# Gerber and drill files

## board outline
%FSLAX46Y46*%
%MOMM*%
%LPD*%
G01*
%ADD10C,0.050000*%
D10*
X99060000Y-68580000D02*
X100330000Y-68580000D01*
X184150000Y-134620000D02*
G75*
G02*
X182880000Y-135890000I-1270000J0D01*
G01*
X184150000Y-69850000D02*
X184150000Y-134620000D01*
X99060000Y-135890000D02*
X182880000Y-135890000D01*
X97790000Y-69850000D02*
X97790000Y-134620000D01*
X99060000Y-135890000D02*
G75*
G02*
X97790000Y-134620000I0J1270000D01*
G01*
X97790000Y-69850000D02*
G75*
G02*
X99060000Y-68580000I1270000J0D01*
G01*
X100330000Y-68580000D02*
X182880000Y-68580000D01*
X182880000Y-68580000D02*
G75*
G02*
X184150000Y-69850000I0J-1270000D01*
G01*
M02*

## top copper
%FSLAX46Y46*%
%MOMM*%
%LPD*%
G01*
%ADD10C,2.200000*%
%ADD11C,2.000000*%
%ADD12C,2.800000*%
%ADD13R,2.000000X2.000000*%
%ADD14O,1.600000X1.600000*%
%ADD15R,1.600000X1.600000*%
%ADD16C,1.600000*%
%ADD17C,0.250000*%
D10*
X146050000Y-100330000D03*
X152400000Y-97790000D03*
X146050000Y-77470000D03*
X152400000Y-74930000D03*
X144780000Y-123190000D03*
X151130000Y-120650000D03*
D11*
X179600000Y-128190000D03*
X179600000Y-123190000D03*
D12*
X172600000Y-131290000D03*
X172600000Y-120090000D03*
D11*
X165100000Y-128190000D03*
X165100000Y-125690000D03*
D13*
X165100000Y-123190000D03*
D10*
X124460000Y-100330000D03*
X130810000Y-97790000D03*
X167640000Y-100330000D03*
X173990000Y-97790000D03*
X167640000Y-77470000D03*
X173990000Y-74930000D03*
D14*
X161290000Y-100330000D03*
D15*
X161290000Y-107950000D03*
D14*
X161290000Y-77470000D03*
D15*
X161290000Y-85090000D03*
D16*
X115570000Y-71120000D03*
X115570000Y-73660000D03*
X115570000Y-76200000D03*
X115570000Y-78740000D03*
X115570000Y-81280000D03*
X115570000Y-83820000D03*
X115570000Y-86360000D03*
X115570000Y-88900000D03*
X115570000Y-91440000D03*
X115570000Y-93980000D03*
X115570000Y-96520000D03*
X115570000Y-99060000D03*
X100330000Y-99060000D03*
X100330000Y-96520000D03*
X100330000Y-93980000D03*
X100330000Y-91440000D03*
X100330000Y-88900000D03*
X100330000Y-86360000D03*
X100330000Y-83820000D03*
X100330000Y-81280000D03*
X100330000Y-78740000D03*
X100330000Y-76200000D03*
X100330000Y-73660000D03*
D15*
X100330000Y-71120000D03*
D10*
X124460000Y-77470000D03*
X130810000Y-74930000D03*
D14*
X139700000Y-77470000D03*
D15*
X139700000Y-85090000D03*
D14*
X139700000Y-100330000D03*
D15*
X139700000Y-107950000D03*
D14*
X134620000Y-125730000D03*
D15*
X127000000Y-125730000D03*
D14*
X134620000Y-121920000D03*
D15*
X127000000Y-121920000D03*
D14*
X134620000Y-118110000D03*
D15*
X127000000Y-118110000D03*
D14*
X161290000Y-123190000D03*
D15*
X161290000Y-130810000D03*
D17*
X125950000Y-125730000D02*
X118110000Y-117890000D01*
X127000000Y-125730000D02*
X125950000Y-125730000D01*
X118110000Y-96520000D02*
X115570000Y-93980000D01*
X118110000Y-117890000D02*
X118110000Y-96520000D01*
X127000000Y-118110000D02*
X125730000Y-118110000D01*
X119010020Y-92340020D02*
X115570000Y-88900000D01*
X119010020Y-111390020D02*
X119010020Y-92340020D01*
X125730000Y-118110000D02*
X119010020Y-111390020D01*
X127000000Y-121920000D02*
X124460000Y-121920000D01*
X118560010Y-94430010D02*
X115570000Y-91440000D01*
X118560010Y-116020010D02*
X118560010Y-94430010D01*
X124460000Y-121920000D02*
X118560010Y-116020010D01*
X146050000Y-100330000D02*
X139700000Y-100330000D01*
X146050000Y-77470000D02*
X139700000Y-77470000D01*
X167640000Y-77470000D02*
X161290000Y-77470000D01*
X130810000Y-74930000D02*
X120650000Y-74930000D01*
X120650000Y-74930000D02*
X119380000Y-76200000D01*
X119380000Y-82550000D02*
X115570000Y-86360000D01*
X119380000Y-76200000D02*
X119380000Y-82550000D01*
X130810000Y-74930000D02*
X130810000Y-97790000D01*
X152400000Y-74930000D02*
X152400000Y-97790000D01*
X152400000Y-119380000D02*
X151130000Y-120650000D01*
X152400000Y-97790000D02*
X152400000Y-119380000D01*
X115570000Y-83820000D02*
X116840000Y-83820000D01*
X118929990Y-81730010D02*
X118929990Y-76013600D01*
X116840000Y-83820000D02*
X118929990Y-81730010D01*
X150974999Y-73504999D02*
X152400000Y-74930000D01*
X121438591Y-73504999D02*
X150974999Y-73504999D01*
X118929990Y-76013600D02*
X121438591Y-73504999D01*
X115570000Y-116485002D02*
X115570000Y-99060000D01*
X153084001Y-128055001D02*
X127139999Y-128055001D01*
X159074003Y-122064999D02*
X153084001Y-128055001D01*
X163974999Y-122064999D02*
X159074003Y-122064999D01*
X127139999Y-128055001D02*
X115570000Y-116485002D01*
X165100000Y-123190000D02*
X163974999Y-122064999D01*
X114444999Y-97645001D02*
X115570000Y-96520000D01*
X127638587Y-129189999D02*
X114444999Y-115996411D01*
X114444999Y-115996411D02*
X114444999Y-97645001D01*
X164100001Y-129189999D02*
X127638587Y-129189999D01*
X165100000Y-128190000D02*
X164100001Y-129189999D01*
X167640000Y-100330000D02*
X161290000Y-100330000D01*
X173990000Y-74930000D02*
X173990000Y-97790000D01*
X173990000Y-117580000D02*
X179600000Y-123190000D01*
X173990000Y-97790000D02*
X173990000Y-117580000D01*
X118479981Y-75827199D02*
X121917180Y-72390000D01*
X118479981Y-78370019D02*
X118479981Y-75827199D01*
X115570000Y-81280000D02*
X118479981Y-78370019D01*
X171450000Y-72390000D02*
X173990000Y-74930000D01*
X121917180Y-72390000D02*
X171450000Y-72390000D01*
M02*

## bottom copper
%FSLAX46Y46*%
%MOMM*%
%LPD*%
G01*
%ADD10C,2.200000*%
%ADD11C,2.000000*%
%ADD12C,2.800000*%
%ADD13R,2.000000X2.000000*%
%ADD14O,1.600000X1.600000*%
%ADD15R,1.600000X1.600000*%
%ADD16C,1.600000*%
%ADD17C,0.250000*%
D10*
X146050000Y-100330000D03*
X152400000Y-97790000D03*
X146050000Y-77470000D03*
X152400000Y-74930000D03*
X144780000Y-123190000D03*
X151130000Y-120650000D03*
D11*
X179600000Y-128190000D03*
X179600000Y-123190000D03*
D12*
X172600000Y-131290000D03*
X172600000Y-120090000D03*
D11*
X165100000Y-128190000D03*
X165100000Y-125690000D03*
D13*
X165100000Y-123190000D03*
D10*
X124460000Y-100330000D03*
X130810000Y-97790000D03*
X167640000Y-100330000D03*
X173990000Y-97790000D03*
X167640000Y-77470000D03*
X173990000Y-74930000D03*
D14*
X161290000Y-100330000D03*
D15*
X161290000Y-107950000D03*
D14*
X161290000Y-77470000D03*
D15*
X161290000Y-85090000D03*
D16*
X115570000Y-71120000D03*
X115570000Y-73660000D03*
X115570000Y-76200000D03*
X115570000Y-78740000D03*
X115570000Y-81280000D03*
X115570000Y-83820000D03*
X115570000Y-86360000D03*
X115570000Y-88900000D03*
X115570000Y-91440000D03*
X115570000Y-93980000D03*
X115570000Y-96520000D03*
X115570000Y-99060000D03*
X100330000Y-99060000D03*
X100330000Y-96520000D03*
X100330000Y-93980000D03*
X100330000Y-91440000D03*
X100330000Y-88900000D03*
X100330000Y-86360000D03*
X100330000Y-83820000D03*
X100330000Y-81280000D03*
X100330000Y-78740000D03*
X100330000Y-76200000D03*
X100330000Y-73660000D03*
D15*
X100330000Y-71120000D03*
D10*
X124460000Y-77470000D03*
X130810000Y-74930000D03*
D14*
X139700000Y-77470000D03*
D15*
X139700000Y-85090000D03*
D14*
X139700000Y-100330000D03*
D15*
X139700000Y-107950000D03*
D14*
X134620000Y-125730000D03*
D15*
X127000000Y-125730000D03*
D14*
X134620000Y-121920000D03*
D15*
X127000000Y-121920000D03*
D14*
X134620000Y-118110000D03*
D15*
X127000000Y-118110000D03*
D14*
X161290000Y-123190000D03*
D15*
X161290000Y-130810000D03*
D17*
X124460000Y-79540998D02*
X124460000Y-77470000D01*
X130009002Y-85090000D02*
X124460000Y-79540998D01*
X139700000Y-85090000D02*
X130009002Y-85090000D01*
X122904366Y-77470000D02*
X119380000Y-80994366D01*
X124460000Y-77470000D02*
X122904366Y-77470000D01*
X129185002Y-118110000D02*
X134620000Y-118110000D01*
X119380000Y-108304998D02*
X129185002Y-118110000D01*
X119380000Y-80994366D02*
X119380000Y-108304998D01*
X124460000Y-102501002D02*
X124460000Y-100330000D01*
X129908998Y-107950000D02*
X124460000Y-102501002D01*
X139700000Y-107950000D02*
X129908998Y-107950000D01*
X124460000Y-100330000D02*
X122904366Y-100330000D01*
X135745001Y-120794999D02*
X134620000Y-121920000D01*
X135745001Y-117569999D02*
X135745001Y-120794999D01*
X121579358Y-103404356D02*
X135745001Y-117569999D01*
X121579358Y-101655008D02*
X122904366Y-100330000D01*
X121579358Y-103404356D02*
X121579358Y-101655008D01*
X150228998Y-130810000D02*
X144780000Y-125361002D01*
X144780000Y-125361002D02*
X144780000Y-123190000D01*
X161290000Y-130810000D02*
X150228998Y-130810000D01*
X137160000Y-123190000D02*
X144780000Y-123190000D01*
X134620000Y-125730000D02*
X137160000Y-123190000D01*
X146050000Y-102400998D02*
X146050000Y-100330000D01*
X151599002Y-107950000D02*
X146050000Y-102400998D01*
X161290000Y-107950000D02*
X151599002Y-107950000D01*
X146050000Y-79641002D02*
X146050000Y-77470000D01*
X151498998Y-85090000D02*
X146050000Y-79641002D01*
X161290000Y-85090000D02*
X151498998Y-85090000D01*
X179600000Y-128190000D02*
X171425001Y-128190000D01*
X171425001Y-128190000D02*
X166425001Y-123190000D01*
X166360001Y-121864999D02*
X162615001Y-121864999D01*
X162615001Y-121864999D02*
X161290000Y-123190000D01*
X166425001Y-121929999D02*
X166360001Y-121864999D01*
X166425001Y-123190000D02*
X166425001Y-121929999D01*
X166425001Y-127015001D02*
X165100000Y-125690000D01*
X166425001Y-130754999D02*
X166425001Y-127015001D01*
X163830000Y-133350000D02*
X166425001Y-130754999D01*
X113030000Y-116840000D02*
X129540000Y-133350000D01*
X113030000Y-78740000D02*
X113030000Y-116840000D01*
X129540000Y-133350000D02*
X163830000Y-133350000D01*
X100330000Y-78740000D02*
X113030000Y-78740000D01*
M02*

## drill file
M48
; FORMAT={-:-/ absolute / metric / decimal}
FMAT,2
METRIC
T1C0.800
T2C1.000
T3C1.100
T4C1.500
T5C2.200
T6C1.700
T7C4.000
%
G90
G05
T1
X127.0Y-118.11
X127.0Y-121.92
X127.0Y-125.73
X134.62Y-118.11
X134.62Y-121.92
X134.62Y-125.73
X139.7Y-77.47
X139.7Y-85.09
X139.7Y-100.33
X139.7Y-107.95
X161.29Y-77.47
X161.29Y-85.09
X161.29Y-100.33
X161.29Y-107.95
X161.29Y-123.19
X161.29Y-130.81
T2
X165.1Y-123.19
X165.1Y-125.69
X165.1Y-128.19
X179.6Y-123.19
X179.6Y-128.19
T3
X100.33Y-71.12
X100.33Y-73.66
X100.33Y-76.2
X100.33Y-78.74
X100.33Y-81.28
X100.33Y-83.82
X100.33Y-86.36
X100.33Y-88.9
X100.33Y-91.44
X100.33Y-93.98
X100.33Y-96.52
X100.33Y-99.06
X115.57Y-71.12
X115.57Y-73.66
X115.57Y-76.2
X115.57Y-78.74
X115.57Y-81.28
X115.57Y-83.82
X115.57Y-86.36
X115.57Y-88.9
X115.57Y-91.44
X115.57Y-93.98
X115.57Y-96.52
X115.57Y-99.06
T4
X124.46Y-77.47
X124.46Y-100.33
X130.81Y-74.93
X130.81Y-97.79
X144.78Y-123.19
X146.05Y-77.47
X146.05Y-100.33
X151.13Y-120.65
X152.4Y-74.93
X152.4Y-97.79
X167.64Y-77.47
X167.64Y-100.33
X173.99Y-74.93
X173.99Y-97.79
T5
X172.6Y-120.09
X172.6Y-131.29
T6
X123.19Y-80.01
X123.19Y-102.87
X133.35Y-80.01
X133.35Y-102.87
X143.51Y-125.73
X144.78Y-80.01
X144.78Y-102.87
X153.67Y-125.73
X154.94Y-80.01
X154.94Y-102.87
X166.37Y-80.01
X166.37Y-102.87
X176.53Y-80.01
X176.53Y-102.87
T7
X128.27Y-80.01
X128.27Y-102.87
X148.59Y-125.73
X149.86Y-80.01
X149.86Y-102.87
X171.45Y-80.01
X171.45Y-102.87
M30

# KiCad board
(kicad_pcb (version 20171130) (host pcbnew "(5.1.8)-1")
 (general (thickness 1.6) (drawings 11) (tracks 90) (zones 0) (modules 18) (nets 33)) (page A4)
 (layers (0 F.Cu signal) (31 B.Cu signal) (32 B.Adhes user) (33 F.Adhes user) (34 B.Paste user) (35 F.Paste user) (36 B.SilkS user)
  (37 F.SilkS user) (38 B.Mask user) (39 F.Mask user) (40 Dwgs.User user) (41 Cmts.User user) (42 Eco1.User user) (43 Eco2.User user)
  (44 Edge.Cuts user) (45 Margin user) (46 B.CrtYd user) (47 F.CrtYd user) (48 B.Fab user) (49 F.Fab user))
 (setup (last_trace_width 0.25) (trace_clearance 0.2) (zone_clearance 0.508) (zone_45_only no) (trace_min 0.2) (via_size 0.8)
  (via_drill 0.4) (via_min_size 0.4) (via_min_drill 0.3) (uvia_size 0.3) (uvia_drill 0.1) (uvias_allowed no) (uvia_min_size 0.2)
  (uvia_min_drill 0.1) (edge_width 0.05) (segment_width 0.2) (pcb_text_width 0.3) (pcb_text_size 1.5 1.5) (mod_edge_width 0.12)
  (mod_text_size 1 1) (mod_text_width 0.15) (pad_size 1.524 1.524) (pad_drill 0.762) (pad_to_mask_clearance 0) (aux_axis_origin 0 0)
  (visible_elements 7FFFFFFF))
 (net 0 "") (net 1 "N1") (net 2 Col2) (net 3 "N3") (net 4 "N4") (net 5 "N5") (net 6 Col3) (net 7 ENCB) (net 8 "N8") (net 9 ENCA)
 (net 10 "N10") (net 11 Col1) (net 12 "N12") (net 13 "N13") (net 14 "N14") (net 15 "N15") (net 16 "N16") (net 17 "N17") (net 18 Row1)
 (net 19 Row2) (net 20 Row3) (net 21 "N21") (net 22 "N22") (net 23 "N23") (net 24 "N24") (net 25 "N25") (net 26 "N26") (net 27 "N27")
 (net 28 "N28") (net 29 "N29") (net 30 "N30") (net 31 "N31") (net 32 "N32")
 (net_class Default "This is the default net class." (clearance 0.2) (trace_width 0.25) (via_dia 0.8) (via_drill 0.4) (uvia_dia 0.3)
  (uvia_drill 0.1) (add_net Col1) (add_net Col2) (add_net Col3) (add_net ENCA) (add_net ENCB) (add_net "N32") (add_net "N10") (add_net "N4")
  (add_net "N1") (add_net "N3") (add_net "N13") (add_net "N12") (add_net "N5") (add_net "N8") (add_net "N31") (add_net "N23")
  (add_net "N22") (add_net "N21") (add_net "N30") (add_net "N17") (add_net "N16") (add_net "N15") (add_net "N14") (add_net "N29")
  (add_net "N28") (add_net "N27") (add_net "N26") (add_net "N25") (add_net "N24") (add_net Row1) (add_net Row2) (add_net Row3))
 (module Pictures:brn (layer F.Cu) (at 110.49 128.27)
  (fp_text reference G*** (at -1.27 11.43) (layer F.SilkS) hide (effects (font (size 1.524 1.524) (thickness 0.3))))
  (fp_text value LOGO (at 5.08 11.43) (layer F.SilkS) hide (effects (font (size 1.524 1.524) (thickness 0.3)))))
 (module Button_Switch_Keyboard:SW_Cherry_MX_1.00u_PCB (layer F.Cu) (at 152.4 97.79)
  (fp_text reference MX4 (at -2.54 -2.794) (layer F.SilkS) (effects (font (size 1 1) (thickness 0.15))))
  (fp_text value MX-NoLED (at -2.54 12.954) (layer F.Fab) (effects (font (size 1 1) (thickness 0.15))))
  (pad "" np_thru_hole circle (at 2.54 5.08) (size 1.7 1.7) (drill 1.7) (layers *.Cu *.Mask))
  (pad "" np_thru_hole circle (at -7.62 5.08) (size 1.7 1.7) (drill 1.7) (layers *.Cu *.Mask))
  (pad "" np_thru_hole circle (at -2.54 5.08) (size 4 4) (drill 4) (layers *.Cu *.Mask))
  (pad 2 thru_hole circle (at -6.35 2.54) (size 2.2 2.2) (drill 1.5) (layers *.Cu *.Mask) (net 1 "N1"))
  (pad 1 thru_hole circle (at 0 0) (size 2.2 2.2) (drill 1.5) (layers *.Cu *.Mask) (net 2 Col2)))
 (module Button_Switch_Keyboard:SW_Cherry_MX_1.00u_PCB (layer F.Cu) (at 152.4 74.93)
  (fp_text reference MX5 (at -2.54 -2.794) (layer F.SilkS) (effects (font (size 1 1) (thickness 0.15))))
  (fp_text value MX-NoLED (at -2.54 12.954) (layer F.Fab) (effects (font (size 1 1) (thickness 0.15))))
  (pad "" np_thru_hole circle (at 2.54 5.08) (size 1.7 1.7) (drill 1.7) (layers *.Cu *.Mask))
  (pad "" np_thru_hole circle (at -7.62 5.08) (size 1.7 1.7) (drill 1.7) (layers *.Cu *.Mask))
  (pad "" np_thru_hole circle (at -2.54 5.08) (size 4 4) (drill 4) (layers *.Cu *.Mask))
  (pad 2 thru_hole circle (at -6.35 2.54) (size 2.2 2.2) (drill 1.5) (layers *.Cu *.Mask) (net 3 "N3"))
  (pad 1 thru_hole circle (at 0 0) (size 2.2 2.2) (drill 1.5) (layers *.Cu *.Mask) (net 2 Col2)))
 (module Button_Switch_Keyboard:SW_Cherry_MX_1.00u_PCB (layer F.Cu) (at 151.13 120.65)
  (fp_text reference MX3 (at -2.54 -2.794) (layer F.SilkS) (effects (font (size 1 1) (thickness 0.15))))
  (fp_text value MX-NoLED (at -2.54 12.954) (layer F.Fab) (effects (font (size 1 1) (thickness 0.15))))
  (pad "" np_thru_hole circle (at 2.54 5.08) (size 1.7 1.7) (drill 1.7) (layers *.Cu *.Mask))
  (pad "" np_thru_hole circle (at -7.62 5.08) (size 1.7 1.7) (drill 1.7) (layers *.Cu *.Mask))
  (pad "" np_thru_hole circle (at -2.54 5.08) (size 4 4) (drill 4) (layers *.Cu *.Mask))
  (pad 2 thru_hole circle (at -6.35 2.54) (size 2.2 2.2) (drill 1.5) (layers *.Cu *.Mask) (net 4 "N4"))
  (pad 1 thru_hole circle (at 0 0) (size 2.2 2.2) (drill 1.5) (layers *.Cu *.Mask) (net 2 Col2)))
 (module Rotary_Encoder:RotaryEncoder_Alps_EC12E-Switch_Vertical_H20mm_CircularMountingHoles (layer F.Cu) (at 165.1 123.19)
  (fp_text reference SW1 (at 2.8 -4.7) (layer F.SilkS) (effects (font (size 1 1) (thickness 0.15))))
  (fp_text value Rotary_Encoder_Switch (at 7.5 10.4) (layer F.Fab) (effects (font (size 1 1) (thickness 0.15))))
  (pad S2 thru_hole circle (at 14.5 5) (size 2 2) (drill 1) (layers *.Cu *.Mask) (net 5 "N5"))
  (pad S1 thru_hole circle (at 14.5 0) (size 2 2) (drill 1) (layers *.Cu *.Mask) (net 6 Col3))
  (pad MP thru_hole circle (at 7.5 8.1) (size 2.8 2.8) (drill 2.2) (layers *.Cu *.Mask))
  (pad MP thru_hole circle (at 7.5 -3.1) (size 2.8 2.8) (drill 2.2) (layers *.Cu *.Mask))
  (pad B thru_hole circle (at 0 5) (size 2 2) (drill 1) (layers *.Cu *.Mask) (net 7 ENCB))
  (pad C thru_hole circle (at 0 2.5) (size 2 2) (drill 1) (layers *.Cu *.Mask) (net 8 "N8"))
  (pad A thru_hole rect (at 0 0) (size 2 2) (drill 1) (layers *.Cu *.Mask) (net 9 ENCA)))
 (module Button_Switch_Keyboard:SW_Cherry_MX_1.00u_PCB (layer F.Cu) (at 130.81 97.79)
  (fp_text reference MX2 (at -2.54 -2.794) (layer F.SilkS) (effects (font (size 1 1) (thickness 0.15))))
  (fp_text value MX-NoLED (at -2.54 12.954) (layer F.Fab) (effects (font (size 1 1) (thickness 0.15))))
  (pad "" np_thru_hole circle (at 2.54 5.08) (size 1.7 1.7) (drill 1.7) (layers *.Cu *.Mask))
  (pad "" np_thru_hole circle (at -7.62 5.08) (size 1.7 1.7) (drill 1.7) (layers *.Cu *.Mask))
  (pad "" np_thru_hole circle (at -2.54 5.08) (size 4 4) (drill 4) (layers *.Cu *.Mask))
  (pad 2 thru_hole circle (at -6.35 2.54) (size 2.2 2.2) (drill 1.5) (layers *.Cu *.Mask) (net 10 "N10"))
  (pad 1 thru_hole circle (at 0 0) (size 2.2 2.2) (drill 1.5) (layers *.Cu *.Mask) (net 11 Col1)))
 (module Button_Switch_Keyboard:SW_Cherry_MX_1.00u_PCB (layer F.Cu) (at 173.99 97.79)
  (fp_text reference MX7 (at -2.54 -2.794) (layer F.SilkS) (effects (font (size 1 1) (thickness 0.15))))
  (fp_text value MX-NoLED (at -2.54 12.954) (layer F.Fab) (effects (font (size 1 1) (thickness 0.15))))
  (pad "" np_thru_hole circle (at 2.54 5.08) (size 1.7 1.7) (drill 1.7) (layers *.Cu *.Mask))
  (pad "" np_thru_hole circle (at -7.62 5.08) (size 1.7 1.7) (drill 1.7) (layers *.Cu *.Mask))
  (pad "" np_thru_hole circle (at -2.54 5.08) (size 4 4) (drill 4) (layers *.Cu *.Mask))
  (pad 2 thru_hole circle (at -6.35 2.54) (size 2.2 2.2) (drill 1.5) (layers *.Cu *.Mask) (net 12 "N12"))
  (pad 1 thru_hole circle (at 0 0) (size 2.2 2.2) (drill 1.5) (layers *.Cu *.Mask) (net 6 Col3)))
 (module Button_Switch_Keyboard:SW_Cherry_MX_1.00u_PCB (layer F.Cu) (at 173.99 74.93)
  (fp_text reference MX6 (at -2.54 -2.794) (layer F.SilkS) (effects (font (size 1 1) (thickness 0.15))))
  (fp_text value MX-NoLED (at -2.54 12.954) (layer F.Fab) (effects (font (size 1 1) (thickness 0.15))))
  (pad "" np_thru_hole circle (at 2.54 5.08) (size 1.7 1.7) (drill 1.7) (layers *.Cu *.Mask))
  (pad "" np_thru_hole circle (at -7.62 5.08) (size 1.7 1.7) (drill 1.7) (layers *.Cu *.Mask))
  (pad "" np_thru_hole circle (at -2.54 5.08) (size 4 4) (drill 4) (layers *.Cu *.Mask))
  (pad 2 thru_hole circle (at -6.35 2.54) (size 2.2 2.2) (drill 1.5) (layers *.Cu *.Mask) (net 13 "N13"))
  (pad 1 thru_hole circle (at 0 0) (size 2.2 2.2) (drill 1.5) (layers *.Cu *.Mask) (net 6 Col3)))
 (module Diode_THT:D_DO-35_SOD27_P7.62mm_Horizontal (layer F.Cu) (at 161.29 107.95 90)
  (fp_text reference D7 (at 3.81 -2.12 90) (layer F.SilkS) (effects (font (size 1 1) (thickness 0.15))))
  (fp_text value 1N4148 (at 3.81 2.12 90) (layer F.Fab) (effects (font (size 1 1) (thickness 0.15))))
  (pad 2 thru_hole oval (at 7.62 0 90) (size 1.6 1.6) (drill 0.8) (layers *.Cu *.Mask) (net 12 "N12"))
  (pad 1 thru_hole rect (at 0 0 90) (size 1.6 1.6) (drill 0.8) (layers *.Cu *.Mask) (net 1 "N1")))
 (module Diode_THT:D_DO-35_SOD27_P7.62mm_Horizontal (layer F.Cu) (at 161.29 85.09 90)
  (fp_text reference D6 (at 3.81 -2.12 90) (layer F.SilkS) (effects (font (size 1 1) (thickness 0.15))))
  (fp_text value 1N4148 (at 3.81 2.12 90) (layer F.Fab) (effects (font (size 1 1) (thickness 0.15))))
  (pad 2 thru_hole oval (at 7.62 0 90) (size 1.6 1.6) (drill 0.8) (layers *.Cu *.Mask) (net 13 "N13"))
  (pad 1 thru_hole rect (at 0 0 90) (size 1.6 1.6) (drill 0.8) (layers *.Cu *.Mask) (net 3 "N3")))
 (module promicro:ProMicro (layer F.Cu) (at 107.95 85.09 270)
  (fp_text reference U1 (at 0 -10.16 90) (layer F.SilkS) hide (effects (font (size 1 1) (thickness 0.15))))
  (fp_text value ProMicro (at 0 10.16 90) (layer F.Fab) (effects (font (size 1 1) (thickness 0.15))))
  (pad 24 thru_hole circle (at -13.97 -7.62 270) (size 1.6 1.6) (drill 1.1) (layers *.Cu *.Mask F.SilkS) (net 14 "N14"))
  (pad 23 thru_hole circle (at -11.43 -7.62 270) (size 1.6 1.6) (drill 1.1) (layers *.Cu *.Mask F.SilkS) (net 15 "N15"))
  (pad 22 thru_hole circle (at -8.89 -7.62 270) (size 1.6 1.6) (drill 1.1) (layers *.Cu *.Mask F.SilkS) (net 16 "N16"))
  (pad 21 thru_hole circle (at -6.35 -7.62 270) (size 1.6 1.6) (drill 1.1) (layers *.Cu *.Mask F.SilkS) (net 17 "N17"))
  (pad 20 thru_hole circle (at -3.81 -7.62 270) (size 1.6 1.6) (drill 1.1) (layers *.Cu *.Mask F.SilkS) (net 6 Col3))
  (pad 19 thru_hole circle (at -1.27 -7.62 270) (size 1.6 1.6) (drill 1.1) (layers *.Cu *.Mask F.SilkS) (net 2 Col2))
  (pad 18 thru_hole circle (at 1.27 -7.62 270) (size 1.6 1.6) (drill 1.1) (layers *.Cu *.Mask F.SilkS) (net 11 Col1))
  (pad 17 thru_hole circle (at 3.81 -7.62 270) (size 1.6 1.6) (drill 1.1) (layers *.Cu *.Mask F.SilkS) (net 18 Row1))
  (pad 16 thru_hole circle (at 6.35 -7.62 270) (size 1.6 1.6) (drill 1.1) (layers *.Cu *.Mask F.SilkS) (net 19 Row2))
  (pad 15 thru_hole circle (at 8.89 -7.62 270) (size 1.6 1.6) (drill 1.1) (layers *.Cu *.Mask F.SilkS) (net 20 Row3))
  (pad 14 thru_hole circle (at 11.43 -7.62 270) (size 1.6 1.6) (drill 1.1) (layers *.Cu *.Mask F.SilkS) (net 7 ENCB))
  (pad 13 thru_hole circle (at 13.97 -7.62 270) (size 1.6 1.6) (drill 1.1) (layers *.Cu *.Mask F.SilkS) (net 9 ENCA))
  (pad 12 thru_hole circle (at 13.97 7.62 270) (size 1.6 1.6) (drill 1.1) (layers *.Cu *.Mask F.SilkS) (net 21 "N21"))
  (pad 11 thru_hole circle (at 11.43 7.62 270) (size 1.6 1.6) (drill 1.1) (layers *.Cu *.Mask F.SilkS) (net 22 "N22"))
  (pad 10 thru_hole circle (at 8.89 7.62 270) (size 1.6 1.6) (drill 1.1) (layers *.Cu *.Mask F.SilkS) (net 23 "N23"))
  (pad 9 thru_hole circle (at 6.35 7.62 270) (size 1.6 1.6) (drill 1.1) (layers *.Cu *.Mask F.SilkS) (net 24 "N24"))
  (pad 8 thru_hole circle (at 3.81 7.62 270) (size 1.6 1.6) (drill 1.1) (layers *.Cu *.Mask F.SilkS) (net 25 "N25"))
  (pad 7 thru_hole circle (at 1.27 7.62 270) (size 1.6 1.6) (drill 1.1) (layers *.Cu *.Mask F.SilkS) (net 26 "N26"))
  (pad 6 thru_hole circle (at -1.27 7.62 270) (size 1.6 1.6) (drill 1.1) (layers *.Cu *.Mask F.SilkS) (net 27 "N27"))
  (pad 5 thru_hole circle (at -3.81 7.62 270) (size 1.6 1.6) (drill 1.1) (layers *.Cu *.Mask F.SilkS) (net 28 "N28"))
  (pad 4 thru_hole circle (at -6.35 7.62 270) (size 1.6 1.6) (drill 1.1) (layers *.Cu *.Mask F.SilkS) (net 8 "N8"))
  (pad 3 thru_hole circle (at -8.89 7.62 270) (size 1.6 1.6) (drill 1.1) (layers *.Cu *.Mask F.SilkS) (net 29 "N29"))
  (pad 2 thru_hole circle (at -11.43 7.62 270) (size 1.6 1.6) (drill 1.1) (layers *.Cu *.Mask F.SilkS) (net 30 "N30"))
  (pad 1 thru_hole rect (at -13.97 7.62 270) (size 1.6 1.6) (drill 1.1) (layers *.Cu *.Mask F.SilkS) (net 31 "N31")))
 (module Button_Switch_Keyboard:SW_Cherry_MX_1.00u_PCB (layer F.Cu) (at 130.81 74.93)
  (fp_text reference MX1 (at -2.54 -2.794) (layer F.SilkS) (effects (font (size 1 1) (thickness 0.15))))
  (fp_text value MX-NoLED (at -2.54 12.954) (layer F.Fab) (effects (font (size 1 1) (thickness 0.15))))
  (pad "" np_thru_hole circle (at 2.54 5.08) (size 1.7 1.7) (drill 1.7) (layers *.Cu *.Mask))
  (pad "" np_thru_hole circle (at -7.62 5.08) (size 1.7 1.7) (drill 1.7) (layers *.Cu *.Mask))
  (pad "" np_thru_hole circle (at -2.54 5.08) (size 4 4) (drill 4) (layers *.Cu *.Mask))
  (pad 2 thru_hole circle (at -6.35 2.54) (size 2.2 2.2) (drill 1.5) (layers *.Cu *.Mask) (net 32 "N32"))
  (pad 1 thru_hole circle (at 0 0) (size 2.2 2.2) (drill 1.5) (layers *.Cu *.Mask) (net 11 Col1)))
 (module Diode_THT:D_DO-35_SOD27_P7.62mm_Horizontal (layer F.Cu) (at 139.7 85.09 90)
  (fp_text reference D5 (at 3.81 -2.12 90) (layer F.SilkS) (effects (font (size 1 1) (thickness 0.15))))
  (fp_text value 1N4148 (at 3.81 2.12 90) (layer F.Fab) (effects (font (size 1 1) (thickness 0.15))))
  (pad 2 thru_hole oval (at 7.62 0 90) (size 1.6 1.6) (drill 0.8) (layers *.Cu *.Mask) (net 3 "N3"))
  (pad 1 thru_hole rect (at 0 0 90) (size 1.6 1.6) (drill 0.8) (layers *.Cu *.Mask) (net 32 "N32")))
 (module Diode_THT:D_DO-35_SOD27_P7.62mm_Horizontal (layer F.Cu) (at 139.7 107.95 90)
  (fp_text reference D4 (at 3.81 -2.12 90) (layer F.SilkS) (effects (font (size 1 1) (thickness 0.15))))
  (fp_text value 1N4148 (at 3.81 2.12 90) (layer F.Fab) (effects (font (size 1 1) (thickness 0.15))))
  (pad 2 thru_hole oval (at 7.62 0 90) (size 1.6 1.6) (drill 0.8) (layers *.Cu *.Mask) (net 1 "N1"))
  (pad 1 thru_hole rect (at 0 0 90) (size 1.6 1.6) (drill 0.8) (layers *.Cu *.Mask) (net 10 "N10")))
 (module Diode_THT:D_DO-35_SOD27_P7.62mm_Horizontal (layer F.Cu) (at 127 125.73)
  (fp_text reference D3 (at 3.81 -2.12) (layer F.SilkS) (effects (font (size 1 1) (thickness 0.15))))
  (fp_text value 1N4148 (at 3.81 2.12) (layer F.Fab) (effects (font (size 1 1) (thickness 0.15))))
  (pad 2 thru_hole oval (at 7.62 0) (size 1.6 1.6) (drill 0.8) (layers *.Cu *.Mask) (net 4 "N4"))
  (pad 1 thru_hole rect (at 0 0) (size 1.6 1.6) (drill 0.8) (layers *.Cu *.Mask) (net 20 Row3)))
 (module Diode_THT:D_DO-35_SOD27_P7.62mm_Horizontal (layer F.Cu) (at 127 121.92)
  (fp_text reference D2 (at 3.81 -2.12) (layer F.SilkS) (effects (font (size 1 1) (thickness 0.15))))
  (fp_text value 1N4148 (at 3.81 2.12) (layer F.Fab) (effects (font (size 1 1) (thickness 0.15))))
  (pad 2 thru_hole oval (at 7.62 0) (size 1.6 1.6) (drill 0.8) (layers *.Cu *.Mask) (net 10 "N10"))
  (pad 1 thru_hole rect (at 0 0) (size 1.6 1.6) (drill 0.8) (layers *.Cu *.Mask) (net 19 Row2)))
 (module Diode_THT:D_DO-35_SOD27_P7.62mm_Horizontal (layer F.Cu) (at 127 118.11)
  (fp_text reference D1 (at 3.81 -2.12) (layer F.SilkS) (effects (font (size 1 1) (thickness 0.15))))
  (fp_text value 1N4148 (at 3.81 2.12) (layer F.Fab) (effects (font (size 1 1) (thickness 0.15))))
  (pad 2 thru_hole oval (at 7.62 0) (size 1.6 1.6) (drill 0.8) (layers *.Cu *.Mask) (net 32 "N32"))
  (pad 1 thru_hole rect (at 0 0) (size 1.6 1.6) (drill 0.8) (layers *.Cu *.Mask) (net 18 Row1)))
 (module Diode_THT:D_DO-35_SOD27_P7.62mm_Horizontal (layer F.Cu) (at 161.29 130.81 90)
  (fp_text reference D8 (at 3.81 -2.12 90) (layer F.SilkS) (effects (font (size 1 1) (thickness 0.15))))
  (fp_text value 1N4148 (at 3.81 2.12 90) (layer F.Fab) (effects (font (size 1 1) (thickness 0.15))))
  (pad 2 thru_hole oval (at 7.62 0 90) (size 1.6 1.6) (drill 0.8) (layers *.Cu *.Mask) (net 5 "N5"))
  (pad 1 thru_hole rect (at 0 0 90) (size 1.6 1.6) (drill 0.8) (layers *.Cu *.Mask) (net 4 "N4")))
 (gr_line (start 99.06 68.58) (end 100.33 68.58) (layer Edge.Cuts) (width 0.05))
 (gr_arc (start 182.88 134.62) (end 182.88 135.89) (angle -90) (layer Edge.Cuts) (width 0.05))
 (gr_line (start 184.15 69.85) (end 184.15 134.62) (layer Edge.Cuts) (width 0.05))
 (gr_line (start 99.06 135.89) (end 182.88 135.89) (layer Edge.Cuts) (width 0.05))
 (gr_line (start 97.79 69.85) (end 97.79 134.62) (layer Edge.Cuts) (width 0.05))
 (gr_arc (start 99.06 134.62) (end 97.79 134.62) (angle -90) (layer Edge.Cuts) (width 0.05))
 (gr_arc (start 99.06 69.85) (end 99.06 68.58) (angle -90) (layer Edge.Cuts) (width 0.05))
 (gr_line (start 100.33 68.58) (end 182.88 68.58) (layer Edge.Cuts) (width 0.05))
 (gr_arc (start 182.88 69.85) (end 184.15 69.85) (angle -90) (layer Edge.Cuts) (width 0.05))
 (segment (start 124.46 79.540998) (end 124.46 77.47) (width 0.25) (layer B.Cu) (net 32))
 (segment (start 130.009002 85.09) (end 124.46 79.540998) (width 0.25) (layer B.Cu) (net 32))
 (segment (start 139.7 85.09) (end 130.009002 85.09) (width 0.25) (layer B.Cu) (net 32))
 (segment (start 122.904366 77.47) (end 119.38 80.994366) (width 0.25) (layer B.Cu) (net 32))
 (segment (start 124.46 77.47) (end 122.904366 77.47) (width 0.25) (layer B.Cu) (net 32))
 (segment (start 129.185002 118.11) (end 134.62 118.11) (width 0.25) (layer B.Cu) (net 32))
 (segment (start 119.38 108.304998) (end 129.185002 118.11) (width 0.25) (layer B.Cu) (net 32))
 (segment (start 119.38 80.994366) (end 119.38 108.304998) (width 0.25) (layer B.Cu) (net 32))
 (segment (start 125.95 125.73) (end 118.11 117.89) (width 0.25) (layer F.Cu) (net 20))
 (segment (start 127 125.73) (end 125.95 125.73) (width 0.25) (layer F.Cu) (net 20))
 (segment (start 118.11 96.52) (end 115.57 93.98) (width 0.25) (layer F.Cu) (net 20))
 (segment (start 118.11 117.89) (end 118.11 96.52) (width 0.25) (layer F.Cu) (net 20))
 (segment (start 124.46 102.501002) (end 124.46 100.33) (width 0.25) (layer B.Cu) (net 10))
 (segment (start 129.908998 107.95) (end 124.46 102.501002) (width 0.25) (layer B.Cu) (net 10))
 (segment (start 139.7 107.95) (end 129.908998 107.95) (width 0.25) (layer B.Cu) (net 10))
 (segment (start 124.46 100.33) (end 122.904366 100.33) (width 0.25) (layer B.Cu) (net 10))
 (segment (start 135.745001 120.794999) (end 134.62 121.92) (width 0.25) (layer B.Cu) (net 10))
 (segment (start 135.745001 117.569999) (end 135.745001 120.794999) (width 0.25) (layer B.Cu) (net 10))
 (segment (start 121.579358 103.404356) (end 135.745001 117.569999) (width 0.25) (layer B.Cu) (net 10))
 (segment (start 121.579358 101.655008) (end 122.904366 100.33) (width 0.25) (layer B.Cu) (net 10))
 (segment (start 121.579358 103.404356) (end 121.579358 101.655008) (width 0.25) (layer B.Cu) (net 10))
 (segment (start 127 118.11) (end 125.73 118.11) (width 0.25) (layer F.Cu) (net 18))
 (segment (start 119.01002 92.34002) (end 115.57 88.9) (width 0.25) (layer F.Cu) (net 18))
 (segment (start 119.01002 111.39002) (end 119.01002 92.34002) (width 0.25) (layer F.Cu) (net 18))
 (segment (start 125.73 118.11) (end 119.01002 111.39002) (width 0.25) (layer F.Cu) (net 18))
 (segment (start 150.228998 130.81) (end 144.78 125.361002) (width 0.25) (layer B.Cu) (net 4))
 (segment (start 144.78 125.361002) (end 144.78 123.19) (width 0.25) (layer B.Cu) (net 4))
 (segment (start 161.29 130.81) (end 150.228998 130.81) (width 0.25) (layer B.Cu) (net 4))
 (segment (start 137.16 123.19) (end 144.78 123.19) (width 0.25) (layer B.Cu) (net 4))
 (segment (start 134.62 125.73) (end 137.16 123.19) (width 0.25) (layer B.Cu) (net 4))
 (segment (start 127 121.92) (end 124.46 121.92) (width 0.25) (layer F.Cu) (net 19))
 (segment (start 118.56001 94.43001) (end 115.57 91.44) (width 0.25) (layer F.Cu) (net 19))
 (segment (start 118.56001 116.02001) (end 118.56001 94.43001) (width 0.25) (layer F.Cu) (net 19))
 (segment (start 124.46 121.92) (end 118.56001 116.02001) (width 0.25) (layer F.Cu) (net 19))
 (segment (start 146.05 102.400998) (end 146.05 100.33) (width 0.25) (layer B.Cu) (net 1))
 (segment (start 151.599002 107.95) (end 146.05 102.400998) (width 0.25) (layer B.Cu) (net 1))
 (segment (start 161.29 107.95) (end 151.599002 107.95) (width 0.25) (layer B.Cu) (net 1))
 (segment (start 146.05 100.33) (end 139.7 100.33) (width 0.25) (layer F.Cu) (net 1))
 (segment (start 146.05 79.641002) (end 146.05 77.47) (width 0.25) (layer B.Cu) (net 3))
 (segment (start 151.498998 85.09) (end 146.05 79.641002) (width 0.25) (layer B.Cu) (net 3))
 (segment (start 161.29 85.09) (end 151.498998 85.09) (width 0.25) (layer B.Cu) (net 3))
 (segment (start 146.05 77.47) (end 139.7 77.47) (width 0.25) (layer F.Cu) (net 3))
 (segment (start 167.64 77.47) (end 161.29 77.47) (width 0.25) (layer F.Cu) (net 13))
 (segment (start 130.81 74.93) (end 120.65 74.93) (width 0.25) (layer F.Cu) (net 11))
 (segment (start 120.65 74.93) (end 119.38 76.2) (width 0.25) (layer F.Cu) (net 11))
 (segment (start 119.38 82.55) (end 115.57 86.36) (width 0.25) (layer F.Cu) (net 11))
 (segment (start 119.38 76.2) (end 119.38 82.55) (width 0.25) (layer F.Cu) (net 11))
 (segment (start 130.81 74.93) (end 130.81 97.79) (width 0.25) (layer F.Cu) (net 11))
 (segment (start 152.4 74.93) (end 152.4 97.79) (width 0.25) (layer F.Cu) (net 2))
 (segment (start 152.4 119.38) (end 151.13 120.65) (width 0.25) (layer F.Cu) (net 2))
 (segment (start 152.4 97.79) (end 152.4 119.38) (width 0.25) (layer F.Cu) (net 2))
 (segment (start 115.57 83.82) (end 116.84 83.82) (width 0.25) (layer F.Cu) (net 2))
 (segment (start 118.92999 81.73001) (end 118.92999 76.0136) (width 0.25) (layer F.Cu) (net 2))
 (segment (start 116.84 83.82) (end 118.92999 81.73001) (width 0.25) (layer F.Cu) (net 2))
 (segment (start 150.974999 73.504999) (end 152.4 74.93) (width 0.25) (layer F.Cu) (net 2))
 (segment (start 121.438591 73.504999) (end 150.974999 73.504999) (width 0.25) (layer F.Cu) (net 2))
 (segment (start 118.92999 76.0136) (end 121.438591 73.504999) (width 0.25) (layer F.Cu) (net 2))
 (segment (start 115.57 116.485002) (end 115.57 99.06) (width 0.25) (layer F.Cu) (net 9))
 (segment (start 153.084001 128.055001) (end 127.139999 128.055001) (width 0.25) (layer F.Cu) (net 9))
 (segment (start 159.074003 122.064999) (end 153.084001 128.055001) (width 0.25) (layer F.Cu) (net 9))
 (segment (start 163.974999 122.064999) (end 159.074003 122.064999) (width 0.25) (layer F.Cu) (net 9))
 (segment (start 127.139999 128.055001) (end 115.57 116.485002) (width 0.25) (layer F.Cu) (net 9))
 (segment (start 165.1 123.19) (end 163.974999 122.064999) (width 0.25) (layer F.Cu) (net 9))
 (segment (start 114.444999 97.645001) (end 115.57 96.52) (width 0.25) (layer F.Cu) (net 7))
 (segment (start 127.638587 129.189999) (end 114.444999 115.996411) (width 0.25) (layer F.Cu) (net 7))
 (segment (start 114.444999 115.996411) (end 114.444999 97.645001) (width 0.25) (layer F.Cu) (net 7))
 (segment (start 164.100001 129.189999) (end 127.638587 129.189999) (width 0.25) (layer F.Cu) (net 7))
 (segment (start 165.1 128.19) (end 164.100001 129.189999) (width 0.25) (layer F.Cu) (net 7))
 (segment (start 167.64 100.33) (end 161.29 100.33) (width 0.25) (layer F.Cu) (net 12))
 (segment (start 179.6 128.19) (end 171.425001 128.19) (width 0.25) (layer B.Cu) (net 5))
 (segment (start 171.425001 128.19) (end 166.425001 123.19) (width 0.25) (layer B.Cu) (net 5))
 (segment (start 166.360001 121.864999) (end 162.615001 121.864999) (width 0.25) (layer B.Cu) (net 5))
 (segment (start 162.615001 121.864999) (end 161.29 123.19) (width 0.25) (layer B.Cu) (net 5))
 (segment (start 166.425001 121.929999) (end 166.360001 121.864999) (width 0.25) (layer B.Cu) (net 5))
 (segment (start 166.425001 123.19) (end 166.425001 121.929999) (width 0.25) (layer B.Cu) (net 5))
 (segment (start 173.99 74.93) (end 173.99 97.79) (width 0.25) (layer F.Cu) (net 6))
 (segment (start 173.99 117.58) (end 179.6 123.19) (width 0.25) (layer F.Cu) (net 6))
 (segment (start 173.99 97.79) (end 173.99 117.58) (width 0.25) (layer F.Cu) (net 6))
 (segment (start 118.479981 75.827199) (end 121.91718 72.39) (width 0.25) (layer F.Cu) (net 6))
 (segment (start 118.479981 78.370019) (end 118.479981 75.827199) (width 0.25) (layer F.Cu) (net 6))
 (segment (start 115.57 81.28) (end 118.479981 78.370019) (width 0.25) (layer F.Cu) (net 6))
 (segment (start 171.45 72.39) (end 173.99 74.93) (width 0.25) (layer F.Cu) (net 6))
 (segment (start 121.91718 72.39) (end 171.45 72.39) (width 0.25) (layer F.Cu) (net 6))
 (segment (start 166.425001 127.015001) (end 165.1 125.69) (width 0.25) (layer B.Cu) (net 8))
 (segment (start 166.425001 130.754999) (end 166.425001 127.015001) (width 0.25) (layer B.Cu) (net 8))
 (segment (start 163.83 133.35) (end 166.425001 130.754999) (width 0.25) (layer B.Cu) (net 8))
 (segment (start 113.03 116.84) (end 129.54 133.35) (width 0.25) (layer B.Cu) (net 8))
 (segment (start 113.03 78.74) (end 113.03 116.84) (width 0.25) (layer B.Cu) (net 8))
 (segment (start 129.54 133.35) (end 163.83 133.35) (width 0.25) (layer B.Cu) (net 8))
 (segment (start 100.33 78.74) (end 113.03 78.74) (width 0.25) (layer B.Cu) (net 8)))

